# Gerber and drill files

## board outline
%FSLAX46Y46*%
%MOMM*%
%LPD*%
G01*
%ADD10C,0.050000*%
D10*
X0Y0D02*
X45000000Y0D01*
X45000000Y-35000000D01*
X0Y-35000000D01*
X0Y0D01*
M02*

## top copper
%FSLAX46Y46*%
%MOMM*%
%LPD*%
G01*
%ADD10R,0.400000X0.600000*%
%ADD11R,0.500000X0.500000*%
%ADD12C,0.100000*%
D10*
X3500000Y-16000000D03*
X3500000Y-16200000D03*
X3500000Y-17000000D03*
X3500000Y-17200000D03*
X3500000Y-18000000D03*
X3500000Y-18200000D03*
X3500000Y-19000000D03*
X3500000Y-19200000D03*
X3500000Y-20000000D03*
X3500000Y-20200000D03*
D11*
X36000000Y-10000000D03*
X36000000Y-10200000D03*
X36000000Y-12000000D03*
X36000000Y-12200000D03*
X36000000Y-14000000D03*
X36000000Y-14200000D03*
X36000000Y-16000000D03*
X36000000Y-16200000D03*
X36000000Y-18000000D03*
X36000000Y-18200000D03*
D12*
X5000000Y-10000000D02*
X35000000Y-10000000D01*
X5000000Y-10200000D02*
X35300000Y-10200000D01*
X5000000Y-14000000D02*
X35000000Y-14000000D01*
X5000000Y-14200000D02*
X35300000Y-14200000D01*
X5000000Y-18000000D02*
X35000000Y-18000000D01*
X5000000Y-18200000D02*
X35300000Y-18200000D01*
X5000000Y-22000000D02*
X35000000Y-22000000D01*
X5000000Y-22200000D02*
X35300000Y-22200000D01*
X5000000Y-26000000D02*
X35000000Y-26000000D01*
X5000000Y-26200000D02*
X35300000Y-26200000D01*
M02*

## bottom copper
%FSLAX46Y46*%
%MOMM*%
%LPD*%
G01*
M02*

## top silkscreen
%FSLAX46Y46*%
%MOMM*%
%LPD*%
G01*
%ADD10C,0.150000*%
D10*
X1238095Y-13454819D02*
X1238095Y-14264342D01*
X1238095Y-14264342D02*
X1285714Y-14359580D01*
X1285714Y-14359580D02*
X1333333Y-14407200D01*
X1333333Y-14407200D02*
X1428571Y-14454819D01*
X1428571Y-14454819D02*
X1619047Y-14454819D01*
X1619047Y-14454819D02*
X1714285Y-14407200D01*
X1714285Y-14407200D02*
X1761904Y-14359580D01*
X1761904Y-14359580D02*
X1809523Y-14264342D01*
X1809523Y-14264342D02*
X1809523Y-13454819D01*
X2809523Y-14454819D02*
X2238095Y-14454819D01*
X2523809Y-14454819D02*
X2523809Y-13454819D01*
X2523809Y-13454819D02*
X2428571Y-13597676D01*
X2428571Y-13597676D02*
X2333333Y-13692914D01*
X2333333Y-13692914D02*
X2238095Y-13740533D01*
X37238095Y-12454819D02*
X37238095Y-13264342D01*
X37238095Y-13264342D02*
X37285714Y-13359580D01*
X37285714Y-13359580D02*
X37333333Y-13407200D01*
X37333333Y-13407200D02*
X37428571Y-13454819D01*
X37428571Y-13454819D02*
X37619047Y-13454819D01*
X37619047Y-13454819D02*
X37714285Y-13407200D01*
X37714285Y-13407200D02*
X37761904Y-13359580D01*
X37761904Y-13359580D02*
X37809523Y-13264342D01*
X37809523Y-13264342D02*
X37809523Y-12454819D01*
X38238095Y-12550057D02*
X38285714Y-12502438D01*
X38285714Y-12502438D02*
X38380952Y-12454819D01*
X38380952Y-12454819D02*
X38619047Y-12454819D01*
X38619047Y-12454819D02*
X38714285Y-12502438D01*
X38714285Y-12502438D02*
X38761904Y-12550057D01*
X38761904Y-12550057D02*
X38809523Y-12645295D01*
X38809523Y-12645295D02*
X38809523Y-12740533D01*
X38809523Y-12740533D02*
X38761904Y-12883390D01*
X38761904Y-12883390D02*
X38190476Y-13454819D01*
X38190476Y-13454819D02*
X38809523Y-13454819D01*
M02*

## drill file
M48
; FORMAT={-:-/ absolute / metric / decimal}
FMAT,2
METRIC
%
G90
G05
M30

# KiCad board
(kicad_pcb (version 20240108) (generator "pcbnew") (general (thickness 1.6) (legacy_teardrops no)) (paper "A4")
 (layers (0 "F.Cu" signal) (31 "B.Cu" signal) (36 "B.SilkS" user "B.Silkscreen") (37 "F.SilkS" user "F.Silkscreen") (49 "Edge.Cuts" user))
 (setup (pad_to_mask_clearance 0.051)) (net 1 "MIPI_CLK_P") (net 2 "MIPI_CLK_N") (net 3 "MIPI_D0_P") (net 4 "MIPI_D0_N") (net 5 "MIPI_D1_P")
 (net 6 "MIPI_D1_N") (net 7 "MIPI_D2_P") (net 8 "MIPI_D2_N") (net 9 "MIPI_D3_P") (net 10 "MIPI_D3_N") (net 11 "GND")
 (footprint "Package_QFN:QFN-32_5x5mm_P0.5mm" (layer "F.Cu") (at 2 18)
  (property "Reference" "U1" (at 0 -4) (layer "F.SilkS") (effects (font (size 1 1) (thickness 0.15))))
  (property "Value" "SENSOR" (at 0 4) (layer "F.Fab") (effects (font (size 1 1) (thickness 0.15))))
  (pad "1" smd rect (at 1.5 -2) (size 0.4 0.6) (layers "F.Cu" "F.Paste" "F.Mask") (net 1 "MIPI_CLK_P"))
  (pad "2" smd rect (at 1.5 -1.8) (size 0.4 0.6) (layers "F.Cu" "F.Paste" "F.Mask") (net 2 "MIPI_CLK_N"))
  (pad "3" smd rect (at 1.5 -1) (size 0.4 0.6) (layers "F.Cu" "F.Paste" "F.Mask") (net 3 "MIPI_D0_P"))
  (pad "4" smd rect (at 1.5 -0.8) (size 0.4 0.6) (layers "F.Cu" "F.Paste" "F.Mask") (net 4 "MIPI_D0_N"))
  (pad "5" smd rect (at 1.5 0) (size 0.4 0.6) (layers "F.Cu" "F.Paste" "F.Mask") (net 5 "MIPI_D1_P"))
  (pad "6" smd rect (at 1.5 0.2) (size 0.4 0.6) (layers "F.Cu" "F.Paste" "F.Mask") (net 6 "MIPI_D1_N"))
  (pad "7" smd rect (at 1.5 1) (size 0.4 0.6) (layers "F.Cu" "F.Paste" "F.Mask") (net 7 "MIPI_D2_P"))
  (pad "8" smd rect (at 1.5 1.2) (size 0.4 0.6) (layers "F.Cu" "F.Paste" "F.Mask") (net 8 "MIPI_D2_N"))
  (pad "9" smd rect (at 1.5 2) (size 0.4 0.6) (layers "F.Cu" "F.Paste" "F.Mask") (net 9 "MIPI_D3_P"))
  (pad "10" smd rect (at 1.5 2.2) (size 0.4 0.6) (layers "F.Cu" "F.Paste" "F.Mask") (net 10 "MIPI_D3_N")))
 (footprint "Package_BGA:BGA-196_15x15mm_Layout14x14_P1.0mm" (layer "F.Cu") (at 38 18)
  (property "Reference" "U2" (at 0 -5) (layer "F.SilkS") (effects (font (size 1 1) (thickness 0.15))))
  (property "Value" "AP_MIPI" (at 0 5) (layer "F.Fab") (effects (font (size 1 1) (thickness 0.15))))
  (pad "A1" smd rect (at -2 -8) (size 0.5 0.5) (layers "F.Cu" "F.Paste" "F.Mask") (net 1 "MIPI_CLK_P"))
  (pad "A2" smd rect (at -2 -7.8) (size 0.5 0.5) (layers "F.Cu" "F.Paste" "F.Mask") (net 2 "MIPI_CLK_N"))
  (pad "B1" smd rect (at -2 -6) (size 0.5 0.5) (layers "F.Cu" "F.Paste" "F.Mask") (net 3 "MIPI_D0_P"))
  (pad "B2" smd rect (at -2 -5.8) (size 0.5 0.5) (layers "F.Cu" "F.Paste" "F.Mask") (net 4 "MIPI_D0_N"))
  (pad "C1" smd rect (at -2 -4) (size 0.5 0.5) (layers "F.Cu" "F.Paste" "F.Mask") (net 5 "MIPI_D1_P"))
  (pad "C2" smd rect (at -2 -3.8) (size 0.5 0.5) (layers "F.Cu" "F.Paste" "F.Mask") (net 6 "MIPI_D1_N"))
  (pad "D1" smd rect (at -2 -2) (size 0.5 0.5) (layers "F.Cu" "F.Paste" "F.Mask") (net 7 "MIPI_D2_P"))
  (pad "D2" smd rect (at -2 -1.8) (size 0.5 0.5) (layers "F.Cu" "F.Paste" "F.Mask") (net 8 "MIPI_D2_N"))
  (pad "E1" smd rect (at -2 0) (size 0.5 0.5) (layers "F.Cu" "F.Paste" "F.Mask") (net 9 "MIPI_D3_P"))
  (pad "E2" smd rect (at -2 0.2) (size 0.5 0.5) (layers "F.Cu" "F.Paste" "F.Mask") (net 10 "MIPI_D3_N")))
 (segment (start 5 10) (end 35 10) (width 0.1) (layer "F.Cu") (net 1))
 (segment (start 5 10.2) (end 35.3 10.2) (width 0.1) (layer "F.Cu") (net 2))
 (segment (start 5 14) (end 35 14) (width 0.1) (layer "F.Cu") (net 3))
 (segment (start 5 14.2) (end 35.3 14.2) (width 0.1) (layer "F.Cu") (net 4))
 (segment (start 5 18) (end 35 18) (width 0.1) (layer "F.Cu") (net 5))
 (segment (start 5 18.2) (end 35.3 18.2) (width 0.1) (layer "F.Cu") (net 6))
 (segment (start 5 22) (end 35 22) (width 0.1) (layer "F.Cu") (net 7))
 (segment (start 5 22.2) (end 35.3 22.2) (width 0.1) (layer "F.Cu") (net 8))
 (segment (start 5 26) (end 35 26) (width 0.1) (layer "F.Cu") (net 9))
 (segment (start 5 26.2) (end 35.3 26.2) (width 0.1) (layer "F.Cu") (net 10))
 (gr_rect (start 0 0) (end 45 35) (layer "Edge.Cuts") (width 0.05)))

